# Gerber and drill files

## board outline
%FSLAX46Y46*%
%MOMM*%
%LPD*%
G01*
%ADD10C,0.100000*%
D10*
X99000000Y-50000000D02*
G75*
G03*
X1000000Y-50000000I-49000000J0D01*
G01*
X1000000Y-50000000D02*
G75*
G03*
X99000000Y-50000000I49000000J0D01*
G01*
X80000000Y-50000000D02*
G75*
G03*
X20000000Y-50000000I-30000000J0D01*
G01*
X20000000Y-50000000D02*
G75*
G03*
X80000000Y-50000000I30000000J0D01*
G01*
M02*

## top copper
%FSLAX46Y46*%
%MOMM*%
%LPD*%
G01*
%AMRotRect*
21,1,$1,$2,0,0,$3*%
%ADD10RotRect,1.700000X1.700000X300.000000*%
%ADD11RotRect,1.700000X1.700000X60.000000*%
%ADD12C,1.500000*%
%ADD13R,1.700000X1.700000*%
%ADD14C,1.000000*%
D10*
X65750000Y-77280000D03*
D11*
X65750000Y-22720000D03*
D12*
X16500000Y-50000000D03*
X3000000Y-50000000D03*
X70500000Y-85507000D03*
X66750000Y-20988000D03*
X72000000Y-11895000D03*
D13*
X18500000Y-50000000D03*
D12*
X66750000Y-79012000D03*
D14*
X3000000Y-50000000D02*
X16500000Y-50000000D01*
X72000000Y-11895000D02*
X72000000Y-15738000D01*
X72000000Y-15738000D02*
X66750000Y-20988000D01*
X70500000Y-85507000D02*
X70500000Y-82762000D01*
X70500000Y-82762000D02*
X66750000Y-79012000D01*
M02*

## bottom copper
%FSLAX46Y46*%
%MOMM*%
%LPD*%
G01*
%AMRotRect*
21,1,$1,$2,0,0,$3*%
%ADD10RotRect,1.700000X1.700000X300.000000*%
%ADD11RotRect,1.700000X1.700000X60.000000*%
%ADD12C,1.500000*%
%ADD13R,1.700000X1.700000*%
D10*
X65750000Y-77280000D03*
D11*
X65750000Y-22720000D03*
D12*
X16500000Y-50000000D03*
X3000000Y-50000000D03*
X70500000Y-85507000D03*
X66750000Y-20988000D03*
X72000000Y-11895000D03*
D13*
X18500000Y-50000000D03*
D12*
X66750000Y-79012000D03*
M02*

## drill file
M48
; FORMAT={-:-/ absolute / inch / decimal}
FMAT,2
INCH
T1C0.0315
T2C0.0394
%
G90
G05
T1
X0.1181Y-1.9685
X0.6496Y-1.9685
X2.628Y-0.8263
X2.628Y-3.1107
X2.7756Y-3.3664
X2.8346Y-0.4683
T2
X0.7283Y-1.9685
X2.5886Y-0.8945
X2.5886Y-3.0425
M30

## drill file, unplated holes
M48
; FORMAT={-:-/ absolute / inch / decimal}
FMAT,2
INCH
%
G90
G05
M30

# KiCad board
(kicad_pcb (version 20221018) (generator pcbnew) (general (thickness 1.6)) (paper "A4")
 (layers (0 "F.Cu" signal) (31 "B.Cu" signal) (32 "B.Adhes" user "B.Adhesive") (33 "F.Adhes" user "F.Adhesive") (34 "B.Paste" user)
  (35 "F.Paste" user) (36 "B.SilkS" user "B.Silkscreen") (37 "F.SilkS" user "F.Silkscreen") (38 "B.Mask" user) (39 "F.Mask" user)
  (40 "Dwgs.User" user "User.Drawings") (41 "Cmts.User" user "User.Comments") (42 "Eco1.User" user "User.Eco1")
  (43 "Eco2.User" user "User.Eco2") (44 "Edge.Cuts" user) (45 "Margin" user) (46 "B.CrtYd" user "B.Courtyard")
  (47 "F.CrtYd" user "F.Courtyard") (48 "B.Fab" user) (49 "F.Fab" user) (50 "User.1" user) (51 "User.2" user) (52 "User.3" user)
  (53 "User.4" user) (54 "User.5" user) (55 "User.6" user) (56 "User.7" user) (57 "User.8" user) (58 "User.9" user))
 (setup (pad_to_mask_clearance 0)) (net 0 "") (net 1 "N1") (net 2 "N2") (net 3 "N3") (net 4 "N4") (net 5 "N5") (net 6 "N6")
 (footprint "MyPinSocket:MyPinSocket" (layer "F.Cu") (at 65.75 77.28 -60)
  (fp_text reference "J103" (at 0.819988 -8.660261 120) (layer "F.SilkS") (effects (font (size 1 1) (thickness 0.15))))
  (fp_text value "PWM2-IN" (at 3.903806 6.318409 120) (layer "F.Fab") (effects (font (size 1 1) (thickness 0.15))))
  (pad "1" thru_hole rect (at 0 0 300) (size 1.7 1.7) (drill 1) (layers "*.Cu" "*.Mask") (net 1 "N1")))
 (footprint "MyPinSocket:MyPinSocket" (layer "F.Cu") (at 65.75 22.72 60)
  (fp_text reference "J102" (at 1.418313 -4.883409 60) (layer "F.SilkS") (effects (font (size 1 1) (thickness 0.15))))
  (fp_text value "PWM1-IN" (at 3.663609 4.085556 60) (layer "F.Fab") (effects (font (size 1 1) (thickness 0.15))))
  (pad "1" thru_hole rect (at 0 0 60) (size 1.7 1.7) (drill 1) (layers "*.Cu" "*.Mask") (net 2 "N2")))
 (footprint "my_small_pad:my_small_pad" (layer "F.Cu") (at 16.5 50)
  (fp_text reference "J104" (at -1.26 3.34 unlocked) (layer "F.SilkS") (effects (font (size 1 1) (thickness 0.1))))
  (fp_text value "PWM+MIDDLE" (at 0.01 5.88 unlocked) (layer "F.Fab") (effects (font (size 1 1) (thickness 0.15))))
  (pad "1" thru_hole circle (at 0 0) (size 1.5 1.5) (drill 0.8) (layers "*.Cu" "*.Mask") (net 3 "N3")))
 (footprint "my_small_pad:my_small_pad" (layer "F.Cu") (at 3 50)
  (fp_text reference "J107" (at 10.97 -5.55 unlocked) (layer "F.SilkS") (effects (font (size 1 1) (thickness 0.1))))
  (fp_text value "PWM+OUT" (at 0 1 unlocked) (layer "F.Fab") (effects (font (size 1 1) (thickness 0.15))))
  (pad "1" thru_hole circle (at 0 0) (size 1.5 1.5) (drill 0.8) (layers "*.Cu" "*.Mask") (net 3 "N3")))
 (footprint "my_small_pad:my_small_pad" (layer "F.Cu") (at 70.5 85.507)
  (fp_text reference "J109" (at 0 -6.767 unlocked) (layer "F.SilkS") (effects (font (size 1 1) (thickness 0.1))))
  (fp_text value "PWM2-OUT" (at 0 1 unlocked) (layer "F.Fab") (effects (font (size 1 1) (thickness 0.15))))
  (pad "1" thru_hole circle (at 0 0) (size 1.5 1.5) (drill 0.8) (layers "*.Cu" "*.Mask") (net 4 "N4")))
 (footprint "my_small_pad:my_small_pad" (layer "F.Cu") (at 66.75 20.988)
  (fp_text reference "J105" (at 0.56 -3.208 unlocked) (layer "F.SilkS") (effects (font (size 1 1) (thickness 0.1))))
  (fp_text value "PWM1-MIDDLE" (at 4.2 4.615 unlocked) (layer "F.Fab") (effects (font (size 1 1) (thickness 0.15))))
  (pad "1" thru_hole circle (at 0 0) (size 1.5 1.5) (drill 0.8) (layers "*.Cu" "*.Mask") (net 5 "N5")))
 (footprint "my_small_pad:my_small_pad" (layer "F.Cu") (at 72 11.895)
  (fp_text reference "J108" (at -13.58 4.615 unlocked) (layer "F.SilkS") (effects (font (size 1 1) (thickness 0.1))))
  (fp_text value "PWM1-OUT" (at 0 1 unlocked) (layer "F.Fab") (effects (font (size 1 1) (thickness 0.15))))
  (pad "1" thru_hole circle (at 0 0) (size 1.5 1.5) (drill 0.8) (layers "*.Cu" "*.Mask") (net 5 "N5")))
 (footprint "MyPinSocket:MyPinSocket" (layer "F.Cu") (at 18.5 50)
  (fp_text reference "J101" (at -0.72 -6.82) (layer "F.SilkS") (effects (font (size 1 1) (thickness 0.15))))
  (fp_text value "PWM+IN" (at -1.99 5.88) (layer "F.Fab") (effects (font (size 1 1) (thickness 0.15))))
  (pad "1" thru_hole rect (at 0 0) (size 1.7 1.7) (drill 1) (layers "*.Cu" "*.Mask") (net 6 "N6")))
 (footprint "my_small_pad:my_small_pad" (layer "F.Cu") (at 66.75 79.012)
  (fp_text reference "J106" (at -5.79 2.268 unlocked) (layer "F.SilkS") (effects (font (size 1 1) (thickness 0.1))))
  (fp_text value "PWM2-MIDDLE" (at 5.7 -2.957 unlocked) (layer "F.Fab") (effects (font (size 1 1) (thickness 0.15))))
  (pad "1" thru_hole circle (at 0 0) (size 1.5 1.5) (drill 0.8) (layers "*.Cu" "*.Mask") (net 4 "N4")))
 (gr_circle (center 50 50) (end 99 50) (stroke (width 0.1) (type default)) (fill none) (layer "Edge.Cuts"))
 (gr_circle (center 50 50) (end 80 50) (stroke (width 0.1) (type default)) (fill none) (layer "Edge.Cuts"))
 (segment (start 3 50) (end 16.5 50) (width 1) (layer "F.Cu") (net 3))
 (segment (start 72 11.895) (end 72 15.738) (width 1) (layer "F.Cu") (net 5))
 (segment (start 72 15.738) (end 66.75 20.988) (width 1) (layer "F.Cu") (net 5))
 (segment (start 70.5 85.507) (end 70.5 82.762) (width 1) (layer "F.Cu") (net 4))
 (segment (start 70.5 82.762) (end 66.75 79.012) (width 1) (layer "F.Cu") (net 4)))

